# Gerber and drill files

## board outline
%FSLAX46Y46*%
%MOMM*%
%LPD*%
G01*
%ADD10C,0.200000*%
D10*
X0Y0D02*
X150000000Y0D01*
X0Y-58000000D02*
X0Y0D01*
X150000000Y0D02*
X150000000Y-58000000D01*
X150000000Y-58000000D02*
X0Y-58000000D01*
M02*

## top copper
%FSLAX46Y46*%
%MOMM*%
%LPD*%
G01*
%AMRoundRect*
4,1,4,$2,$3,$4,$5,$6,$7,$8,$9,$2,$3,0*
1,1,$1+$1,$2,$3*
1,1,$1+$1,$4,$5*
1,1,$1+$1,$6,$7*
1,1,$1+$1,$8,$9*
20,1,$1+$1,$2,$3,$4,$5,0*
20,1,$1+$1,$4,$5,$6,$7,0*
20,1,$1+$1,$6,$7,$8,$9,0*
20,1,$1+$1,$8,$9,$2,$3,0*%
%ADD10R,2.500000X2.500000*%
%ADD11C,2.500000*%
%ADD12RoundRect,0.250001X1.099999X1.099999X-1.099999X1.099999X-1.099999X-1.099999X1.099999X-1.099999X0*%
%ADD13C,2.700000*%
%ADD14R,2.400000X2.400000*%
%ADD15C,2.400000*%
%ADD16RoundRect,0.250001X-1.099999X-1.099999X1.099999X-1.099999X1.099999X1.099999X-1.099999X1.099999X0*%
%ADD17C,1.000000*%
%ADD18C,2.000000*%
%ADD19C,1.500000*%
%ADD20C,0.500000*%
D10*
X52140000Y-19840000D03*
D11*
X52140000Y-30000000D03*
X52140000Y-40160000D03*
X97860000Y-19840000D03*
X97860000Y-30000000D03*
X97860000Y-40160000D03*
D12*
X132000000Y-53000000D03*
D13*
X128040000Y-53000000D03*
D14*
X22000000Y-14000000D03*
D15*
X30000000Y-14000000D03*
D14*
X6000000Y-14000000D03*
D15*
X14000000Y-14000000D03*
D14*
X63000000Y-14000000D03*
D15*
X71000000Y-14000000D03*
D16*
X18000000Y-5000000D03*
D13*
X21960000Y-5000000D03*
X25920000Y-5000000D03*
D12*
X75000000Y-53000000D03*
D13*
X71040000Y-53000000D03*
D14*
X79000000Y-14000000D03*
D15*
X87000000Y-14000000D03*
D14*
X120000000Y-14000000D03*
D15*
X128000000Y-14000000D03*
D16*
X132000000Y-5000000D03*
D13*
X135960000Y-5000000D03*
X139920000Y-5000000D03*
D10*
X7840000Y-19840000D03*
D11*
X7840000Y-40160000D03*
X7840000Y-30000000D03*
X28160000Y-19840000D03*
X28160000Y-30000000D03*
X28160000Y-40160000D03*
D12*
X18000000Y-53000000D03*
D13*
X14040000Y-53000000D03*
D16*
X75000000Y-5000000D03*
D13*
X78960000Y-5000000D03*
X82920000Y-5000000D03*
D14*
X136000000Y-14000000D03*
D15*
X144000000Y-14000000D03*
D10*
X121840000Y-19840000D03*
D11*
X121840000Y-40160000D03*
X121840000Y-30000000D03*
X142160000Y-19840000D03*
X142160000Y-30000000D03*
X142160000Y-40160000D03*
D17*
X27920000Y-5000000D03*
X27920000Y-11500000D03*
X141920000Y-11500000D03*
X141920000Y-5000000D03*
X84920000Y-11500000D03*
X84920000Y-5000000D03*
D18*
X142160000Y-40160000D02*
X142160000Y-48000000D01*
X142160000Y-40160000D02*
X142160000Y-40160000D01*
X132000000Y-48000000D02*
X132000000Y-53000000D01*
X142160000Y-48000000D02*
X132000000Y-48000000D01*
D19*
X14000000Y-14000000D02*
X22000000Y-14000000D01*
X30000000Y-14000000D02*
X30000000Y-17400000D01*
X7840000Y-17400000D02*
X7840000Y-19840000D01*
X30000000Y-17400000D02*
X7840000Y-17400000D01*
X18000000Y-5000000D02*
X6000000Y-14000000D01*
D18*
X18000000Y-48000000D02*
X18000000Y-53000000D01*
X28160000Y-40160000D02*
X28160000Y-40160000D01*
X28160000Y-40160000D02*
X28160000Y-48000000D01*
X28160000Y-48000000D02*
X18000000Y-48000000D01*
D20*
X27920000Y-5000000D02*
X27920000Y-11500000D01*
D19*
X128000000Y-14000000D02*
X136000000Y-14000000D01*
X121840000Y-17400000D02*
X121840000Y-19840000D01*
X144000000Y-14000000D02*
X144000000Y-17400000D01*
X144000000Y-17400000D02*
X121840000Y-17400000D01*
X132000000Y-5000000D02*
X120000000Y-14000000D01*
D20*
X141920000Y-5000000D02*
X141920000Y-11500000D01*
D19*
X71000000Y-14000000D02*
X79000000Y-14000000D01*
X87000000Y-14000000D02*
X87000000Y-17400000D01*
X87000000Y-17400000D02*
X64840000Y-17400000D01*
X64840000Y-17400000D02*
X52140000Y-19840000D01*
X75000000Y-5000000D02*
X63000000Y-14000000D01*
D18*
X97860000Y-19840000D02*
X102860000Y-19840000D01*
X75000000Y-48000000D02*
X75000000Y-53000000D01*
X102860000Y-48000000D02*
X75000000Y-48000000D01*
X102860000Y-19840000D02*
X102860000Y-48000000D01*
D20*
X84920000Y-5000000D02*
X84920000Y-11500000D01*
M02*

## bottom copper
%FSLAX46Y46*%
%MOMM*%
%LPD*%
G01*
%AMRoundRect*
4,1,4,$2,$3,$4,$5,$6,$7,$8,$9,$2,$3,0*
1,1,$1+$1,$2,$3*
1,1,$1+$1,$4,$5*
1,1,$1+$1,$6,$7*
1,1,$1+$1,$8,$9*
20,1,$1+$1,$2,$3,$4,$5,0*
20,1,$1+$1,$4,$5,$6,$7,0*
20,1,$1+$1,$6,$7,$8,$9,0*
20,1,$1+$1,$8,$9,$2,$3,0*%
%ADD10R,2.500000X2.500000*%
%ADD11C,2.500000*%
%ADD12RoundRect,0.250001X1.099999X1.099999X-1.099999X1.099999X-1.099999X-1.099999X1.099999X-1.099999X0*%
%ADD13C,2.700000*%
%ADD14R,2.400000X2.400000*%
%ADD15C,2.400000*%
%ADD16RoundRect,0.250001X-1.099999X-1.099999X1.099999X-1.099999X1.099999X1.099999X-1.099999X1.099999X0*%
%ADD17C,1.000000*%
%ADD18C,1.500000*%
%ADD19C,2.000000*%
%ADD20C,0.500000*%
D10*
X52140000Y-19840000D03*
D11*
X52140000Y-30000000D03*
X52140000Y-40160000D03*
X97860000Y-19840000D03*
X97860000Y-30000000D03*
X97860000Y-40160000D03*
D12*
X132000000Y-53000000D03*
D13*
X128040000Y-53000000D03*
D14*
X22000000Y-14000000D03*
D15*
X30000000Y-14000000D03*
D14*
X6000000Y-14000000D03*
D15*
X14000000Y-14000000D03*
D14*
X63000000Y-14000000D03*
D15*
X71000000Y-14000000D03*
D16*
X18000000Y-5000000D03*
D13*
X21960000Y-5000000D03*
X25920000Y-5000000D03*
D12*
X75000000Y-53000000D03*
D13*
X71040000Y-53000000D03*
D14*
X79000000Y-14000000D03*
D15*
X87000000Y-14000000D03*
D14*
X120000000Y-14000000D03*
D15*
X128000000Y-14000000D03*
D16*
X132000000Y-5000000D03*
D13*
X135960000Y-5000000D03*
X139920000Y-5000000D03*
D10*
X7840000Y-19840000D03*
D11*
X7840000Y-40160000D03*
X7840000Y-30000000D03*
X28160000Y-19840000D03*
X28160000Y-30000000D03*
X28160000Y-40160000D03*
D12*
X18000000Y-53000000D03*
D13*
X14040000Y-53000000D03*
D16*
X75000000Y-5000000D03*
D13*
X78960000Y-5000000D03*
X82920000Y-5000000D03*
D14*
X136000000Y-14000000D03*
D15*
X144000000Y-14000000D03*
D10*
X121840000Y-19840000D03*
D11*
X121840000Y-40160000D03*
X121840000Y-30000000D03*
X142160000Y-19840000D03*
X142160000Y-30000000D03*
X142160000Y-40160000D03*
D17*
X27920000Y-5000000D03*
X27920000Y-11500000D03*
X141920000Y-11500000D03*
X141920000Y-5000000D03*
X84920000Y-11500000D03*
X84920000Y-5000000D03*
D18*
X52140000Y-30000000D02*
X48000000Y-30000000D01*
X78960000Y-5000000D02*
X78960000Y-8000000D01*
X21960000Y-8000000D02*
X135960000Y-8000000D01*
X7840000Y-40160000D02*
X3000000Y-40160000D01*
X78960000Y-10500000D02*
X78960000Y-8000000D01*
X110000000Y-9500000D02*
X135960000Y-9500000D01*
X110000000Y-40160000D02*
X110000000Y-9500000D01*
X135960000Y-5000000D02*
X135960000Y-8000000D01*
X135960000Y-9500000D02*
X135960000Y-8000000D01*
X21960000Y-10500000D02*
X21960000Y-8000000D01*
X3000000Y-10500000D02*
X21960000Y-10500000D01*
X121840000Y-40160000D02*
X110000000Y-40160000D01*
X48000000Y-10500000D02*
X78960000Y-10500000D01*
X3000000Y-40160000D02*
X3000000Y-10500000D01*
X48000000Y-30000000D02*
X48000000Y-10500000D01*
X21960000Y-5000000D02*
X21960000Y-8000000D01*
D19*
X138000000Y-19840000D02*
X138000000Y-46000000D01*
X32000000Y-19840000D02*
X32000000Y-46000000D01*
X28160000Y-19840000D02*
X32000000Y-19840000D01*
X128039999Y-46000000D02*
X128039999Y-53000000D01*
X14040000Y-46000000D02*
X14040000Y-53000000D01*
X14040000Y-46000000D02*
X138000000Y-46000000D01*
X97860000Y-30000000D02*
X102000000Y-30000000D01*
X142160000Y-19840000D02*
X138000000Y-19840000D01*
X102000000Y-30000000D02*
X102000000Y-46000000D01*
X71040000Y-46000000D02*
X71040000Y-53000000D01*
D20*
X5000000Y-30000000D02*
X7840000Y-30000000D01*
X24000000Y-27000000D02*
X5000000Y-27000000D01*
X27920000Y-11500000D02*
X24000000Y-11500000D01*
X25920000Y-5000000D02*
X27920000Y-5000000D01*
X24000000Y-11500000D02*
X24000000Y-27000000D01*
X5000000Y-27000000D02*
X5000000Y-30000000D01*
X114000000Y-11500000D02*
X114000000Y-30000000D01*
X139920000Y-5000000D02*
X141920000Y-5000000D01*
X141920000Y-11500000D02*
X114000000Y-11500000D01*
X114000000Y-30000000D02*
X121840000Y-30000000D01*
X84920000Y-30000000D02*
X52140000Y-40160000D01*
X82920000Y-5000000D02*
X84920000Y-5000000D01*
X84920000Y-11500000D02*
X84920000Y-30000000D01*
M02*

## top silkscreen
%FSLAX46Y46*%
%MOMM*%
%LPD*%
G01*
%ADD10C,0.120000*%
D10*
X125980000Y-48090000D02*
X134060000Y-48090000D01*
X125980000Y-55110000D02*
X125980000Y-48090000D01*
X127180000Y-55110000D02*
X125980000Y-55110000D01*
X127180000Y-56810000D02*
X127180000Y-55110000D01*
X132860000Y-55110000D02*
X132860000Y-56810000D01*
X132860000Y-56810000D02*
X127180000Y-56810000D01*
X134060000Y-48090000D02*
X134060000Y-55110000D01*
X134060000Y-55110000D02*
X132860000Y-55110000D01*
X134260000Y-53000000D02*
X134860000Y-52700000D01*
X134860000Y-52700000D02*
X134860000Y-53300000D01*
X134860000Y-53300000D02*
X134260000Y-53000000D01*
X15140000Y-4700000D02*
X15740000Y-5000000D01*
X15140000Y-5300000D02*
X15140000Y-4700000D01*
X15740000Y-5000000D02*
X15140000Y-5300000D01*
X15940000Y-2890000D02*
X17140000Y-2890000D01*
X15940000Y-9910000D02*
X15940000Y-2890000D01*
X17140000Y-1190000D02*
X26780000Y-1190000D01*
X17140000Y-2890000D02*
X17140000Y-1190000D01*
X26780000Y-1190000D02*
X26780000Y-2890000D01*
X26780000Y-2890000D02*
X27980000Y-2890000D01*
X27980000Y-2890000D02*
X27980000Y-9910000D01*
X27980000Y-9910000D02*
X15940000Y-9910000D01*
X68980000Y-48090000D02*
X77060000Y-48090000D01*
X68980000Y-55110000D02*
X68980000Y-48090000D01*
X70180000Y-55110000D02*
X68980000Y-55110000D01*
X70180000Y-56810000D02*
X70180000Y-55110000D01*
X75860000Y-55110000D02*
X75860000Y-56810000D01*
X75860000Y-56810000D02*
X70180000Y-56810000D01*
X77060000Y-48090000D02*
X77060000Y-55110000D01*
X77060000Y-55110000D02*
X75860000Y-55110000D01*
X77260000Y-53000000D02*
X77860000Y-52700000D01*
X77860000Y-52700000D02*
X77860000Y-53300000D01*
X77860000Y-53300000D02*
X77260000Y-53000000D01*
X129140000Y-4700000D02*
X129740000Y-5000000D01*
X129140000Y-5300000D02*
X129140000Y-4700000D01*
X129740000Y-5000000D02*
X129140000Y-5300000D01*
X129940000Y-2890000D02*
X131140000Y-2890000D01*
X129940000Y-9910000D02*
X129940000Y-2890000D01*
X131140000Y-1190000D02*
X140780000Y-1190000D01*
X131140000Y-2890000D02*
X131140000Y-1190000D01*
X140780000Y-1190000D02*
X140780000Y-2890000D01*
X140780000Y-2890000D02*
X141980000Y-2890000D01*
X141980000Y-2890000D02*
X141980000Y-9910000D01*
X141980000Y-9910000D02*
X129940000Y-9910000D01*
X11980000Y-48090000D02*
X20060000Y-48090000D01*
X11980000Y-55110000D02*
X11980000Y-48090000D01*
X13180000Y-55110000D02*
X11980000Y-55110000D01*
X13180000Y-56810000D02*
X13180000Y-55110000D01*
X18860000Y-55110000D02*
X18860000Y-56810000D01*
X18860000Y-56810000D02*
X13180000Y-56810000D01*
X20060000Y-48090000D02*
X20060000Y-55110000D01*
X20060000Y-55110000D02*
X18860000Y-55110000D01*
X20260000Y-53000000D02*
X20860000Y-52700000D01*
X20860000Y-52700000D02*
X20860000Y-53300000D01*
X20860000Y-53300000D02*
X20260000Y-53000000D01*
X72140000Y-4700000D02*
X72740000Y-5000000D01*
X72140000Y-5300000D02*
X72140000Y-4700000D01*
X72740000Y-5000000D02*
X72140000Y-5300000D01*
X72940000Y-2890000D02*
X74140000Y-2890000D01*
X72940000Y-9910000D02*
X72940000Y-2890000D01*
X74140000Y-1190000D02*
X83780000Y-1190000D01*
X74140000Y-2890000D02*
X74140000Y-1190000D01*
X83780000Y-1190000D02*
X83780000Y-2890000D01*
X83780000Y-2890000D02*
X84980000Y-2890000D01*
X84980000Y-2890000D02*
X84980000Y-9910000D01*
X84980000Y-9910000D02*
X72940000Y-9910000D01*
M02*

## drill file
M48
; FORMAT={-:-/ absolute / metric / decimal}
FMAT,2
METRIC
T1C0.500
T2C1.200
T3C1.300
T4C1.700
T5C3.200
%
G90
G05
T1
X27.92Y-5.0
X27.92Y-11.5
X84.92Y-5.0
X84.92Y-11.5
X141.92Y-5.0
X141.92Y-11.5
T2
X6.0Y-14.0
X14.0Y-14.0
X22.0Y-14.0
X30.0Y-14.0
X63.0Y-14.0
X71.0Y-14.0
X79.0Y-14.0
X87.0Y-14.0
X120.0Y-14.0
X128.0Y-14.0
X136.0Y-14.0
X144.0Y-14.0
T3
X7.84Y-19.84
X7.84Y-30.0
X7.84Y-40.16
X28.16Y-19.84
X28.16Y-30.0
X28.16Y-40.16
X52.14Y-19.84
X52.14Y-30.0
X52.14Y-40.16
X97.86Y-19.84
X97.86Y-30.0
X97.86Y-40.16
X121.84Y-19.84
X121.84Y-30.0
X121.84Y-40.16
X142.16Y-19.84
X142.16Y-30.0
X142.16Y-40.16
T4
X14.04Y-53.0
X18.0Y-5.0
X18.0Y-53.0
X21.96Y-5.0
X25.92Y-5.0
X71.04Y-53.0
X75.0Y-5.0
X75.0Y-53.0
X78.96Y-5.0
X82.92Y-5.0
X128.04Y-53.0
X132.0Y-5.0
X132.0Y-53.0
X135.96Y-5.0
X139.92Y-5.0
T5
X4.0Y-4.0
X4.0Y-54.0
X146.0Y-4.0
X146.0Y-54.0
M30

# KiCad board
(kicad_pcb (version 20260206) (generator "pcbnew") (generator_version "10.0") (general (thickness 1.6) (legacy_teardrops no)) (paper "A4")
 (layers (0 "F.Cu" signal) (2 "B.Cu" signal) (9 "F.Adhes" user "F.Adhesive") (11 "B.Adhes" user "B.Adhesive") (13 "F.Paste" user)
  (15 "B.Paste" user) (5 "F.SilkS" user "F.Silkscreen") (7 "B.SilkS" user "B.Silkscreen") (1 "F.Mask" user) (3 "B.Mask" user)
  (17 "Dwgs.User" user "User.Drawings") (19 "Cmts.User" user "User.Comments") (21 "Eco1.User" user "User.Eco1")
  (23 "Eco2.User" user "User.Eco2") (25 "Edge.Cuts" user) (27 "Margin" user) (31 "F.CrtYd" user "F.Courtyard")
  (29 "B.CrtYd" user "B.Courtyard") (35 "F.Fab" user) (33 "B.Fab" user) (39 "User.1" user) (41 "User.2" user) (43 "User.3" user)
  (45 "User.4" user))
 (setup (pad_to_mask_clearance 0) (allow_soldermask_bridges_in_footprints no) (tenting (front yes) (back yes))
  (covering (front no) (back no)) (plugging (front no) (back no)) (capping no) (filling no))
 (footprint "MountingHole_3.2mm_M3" (layer "F.Cu") (at 4 4)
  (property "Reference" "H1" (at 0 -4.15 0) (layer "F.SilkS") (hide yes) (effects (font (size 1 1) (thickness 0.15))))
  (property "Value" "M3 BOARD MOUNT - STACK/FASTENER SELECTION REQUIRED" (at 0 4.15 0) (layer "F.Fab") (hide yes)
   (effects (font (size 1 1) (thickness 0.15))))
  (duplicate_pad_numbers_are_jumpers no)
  (pad "" np_thru_hole circle (at 0 0) (size 3.2 3.2) (drill 3.2) (layers "*.Cu")))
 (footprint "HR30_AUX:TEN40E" (layer "F.Cu") (at 75 30)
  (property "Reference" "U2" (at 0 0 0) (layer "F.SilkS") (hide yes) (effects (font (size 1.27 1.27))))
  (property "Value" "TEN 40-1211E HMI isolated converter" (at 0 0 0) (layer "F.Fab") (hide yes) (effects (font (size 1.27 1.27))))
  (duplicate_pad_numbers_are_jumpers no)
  (pad "1" thru_hole rect (at -22.86 -10.16) (size 2.5 2.5) (drill 1.3) (layers "*.Cu") (remove_unused_layers no) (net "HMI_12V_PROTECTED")
   (thermal_bridge_angle 45))
  (pad "2" thru_hole circle (at -22.86 0) (size 2.5 2.5) (drill 1.3) (layers "*.Cu") (remove_unused_layers no) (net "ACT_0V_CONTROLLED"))
  (pad "3" thru_hole circle (at -22.86 10.16) (size 2.5 2.5) (drill 1.3) (layers "*.Cu") (remove_unused_layers no) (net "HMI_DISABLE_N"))
  (pad "4" thru_hole circle (at 22.86 -10.16) (size 2.5 2.5) (drill 1.3) (layers "*.Cu") (remove_unused_layers no) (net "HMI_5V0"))
  (pad "5" thru_hole circle (at 22.86 0) (size 2.5 2.5) (drill 1.3) (layers "*.Cu") (remove_unused_layers no) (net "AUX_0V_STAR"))
  (pad "6" thru_hole circle (at 22.86 10.16) (size 2.5 2.5) (drill 1.3) (layers "*.Cu") (remove_unused_layers no)))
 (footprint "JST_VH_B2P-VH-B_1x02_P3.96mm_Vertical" (layer "F.Cu") (at 132 53 180)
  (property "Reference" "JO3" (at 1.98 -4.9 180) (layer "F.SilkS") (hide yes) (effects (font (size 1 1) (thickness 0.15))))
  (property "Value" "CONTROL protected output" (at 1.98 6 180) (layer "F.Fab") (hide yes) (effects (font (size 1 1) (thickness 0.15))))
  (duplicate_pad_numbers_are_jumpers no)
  (fp_line (start 6.02 4.91) (end -2.06 4.91) (stroke (width 0.12) (type solid)) (layer "F.SilkS"))
  (fp_line (start 6.02 -2.11) (end 6.02 4.91) (stroke (width 0.12) (type solid)) (layer "F.SilkS"))
  (fp_line (start 4.82 -2.11) (end 6.02 -2.11) (stroke (width 0.12) (type solid)) (layer "F.SilkS"))
  (fp_line (start 4.82 -3.81) (end 4.82 -2.11) (stroke (width 0.12) (type solid)) (layer "F.SilkS"))
  (fp_line (start -0.86 -2.11) (end -0.86 -3.81) (stroke (width 0.12) (type solid)) (layer "F.SilkS"))
  (fp_line (start -0.86 -3.81) (end 4.82 -3.81) (stroke (width 0.12) (type solid)) (layer "F.SilkS"))
  (fp_line (start -2.06 4.91) (end -2.06 -2.11) (stroke (width 0.12) (type solid)) (layer "F.SilkS"))
  (fp_line (start -2.06 -2.11) (end -0.86 -2.11) (stroke (width 0.12) (type solid)) (layer "F.SilkS"))
  (fp_line (start -2.26 0) (end -2.86 0.3) (stroke (width 0.12) (type solid)) (layer "F.SilkS"))
  (fp_line (start -2.86 0.3) (end -2.86 -0.3) (stroke (width 0.12) (type solid)) (layer "F.SilkS"))
  (fp_line (start -2.86 -0.3) (end -2.26 0) (stroke (width 0.12) (type solid)) (layer "F.SilkS"))
  (pad "1" thru_hole roundrect (at 0 0 180) (size 2.7 2.7) (drill 1.7) (layers "*.Cu") (remove_unused_layers no) (roundrect_rratio 0.092593)
   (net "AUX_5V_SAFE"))
  (pad "2" thru_hole circle (at 3.96 0 180) (size 2.7 2.7) (drill 1.7) (layers "*.Cu") (remove_unused_layers no) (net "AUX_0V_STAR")))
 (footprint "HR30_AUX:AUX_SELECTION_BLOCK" (layer "F.Cu") (at 26 14)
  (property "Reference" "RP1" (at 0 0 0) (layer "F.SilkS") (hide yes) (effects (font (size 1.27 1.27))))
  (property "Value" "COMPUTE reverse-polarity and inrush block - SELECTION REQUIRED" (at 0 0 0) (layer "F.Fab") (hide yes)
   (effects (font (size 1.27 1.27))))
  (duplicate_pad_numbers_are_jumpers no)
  (pad "1" thru_hole rect (at -4 0) (size 2.4 2.4) (drill 1.2) (layers "*.Cu") (remove_unused_layers no) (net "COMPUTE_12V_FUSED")
   (thermal_bridge_angle 45))
  (pad "2" thru_hole circle (at 4 0) (size 2.4 2.4) (drill 1.2) (layers "*.Cu") (remove_unused_layers no) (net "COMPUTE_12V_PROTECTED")))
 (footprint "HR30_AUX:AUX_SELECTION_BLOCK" (layer "F.Cu") (at 10 14)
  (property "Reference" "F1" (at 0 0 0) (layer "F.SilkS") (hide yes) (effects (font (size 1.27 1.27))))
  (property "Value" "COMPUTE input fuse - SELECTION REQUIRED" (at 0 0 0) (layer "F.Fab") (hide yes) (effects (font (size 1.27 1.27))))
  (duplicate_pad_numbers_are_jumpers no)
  (pad "1" thru_hole rect (at -4 0) (size 2.4 2.4) (drill 1.2) (layers "*.Cu") (remove_unused_layers no) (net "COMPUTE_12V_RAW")
   (thermal_bridge_angle 45))
  (pad "2" thru_hole circle (at 4 0) (size 2.4 2.4) (drill 1.2) (layers "*.Cu") (remove_unused_layers no) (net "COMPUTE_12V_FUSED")))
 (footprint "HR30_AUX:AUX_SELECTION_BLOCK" (layer "F.Cu") (at 67 14)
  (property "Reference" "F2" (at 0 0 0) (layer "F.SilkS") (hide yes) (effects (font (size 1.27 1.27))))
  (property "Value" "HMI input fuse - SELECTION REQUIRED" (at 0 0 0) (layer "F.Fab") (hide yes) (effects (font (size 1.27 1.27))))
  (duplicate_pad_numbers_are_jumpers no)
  (pad "1" thru_hole rect (at -4 0) (size 2.4 2.4) (drill 1.2) (layers "*.Cu") (remove_unused_layers no) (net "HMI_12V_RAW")
   (thermal_bridge_angle 45))
  (pad "2" thru_hole circle (at 4 0) (size 2.4 2.4) (drill 1.2) (layers "*.Cu") (remove_unused_layers no) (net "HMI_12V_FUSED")))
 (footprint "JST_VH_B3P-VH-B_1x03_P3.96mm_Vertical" (layer "F.Cu") (at 18 5)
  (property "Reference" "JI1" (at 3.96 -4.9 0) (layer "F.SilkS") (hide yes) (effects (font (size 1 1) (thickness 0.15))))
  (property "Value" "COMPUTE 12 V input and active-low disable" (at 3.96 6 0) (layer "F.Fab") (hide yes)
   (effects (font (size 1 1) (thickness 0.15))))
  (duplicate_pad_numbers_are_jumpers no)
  (fp_line (start -2.86 -0.3) (end -2.26 0) (stroke (width 0.12) (type solid)) (layer "F.SilkS"))
  (fp_line (start -2.86 0.3) (end -2.86 -0.3) (stroke (width 0.12) (type solid)) (layer "F.SilkS"))
  (fp_line (start -2.26 0) (end -2.86 0.3) (stroke (width 0.12) (type solid)) (layer "F.SilkS"))
  (fp_line (start -2.06 -2.11) (end -0.86 -2.11) (stroke (width 0.12) (type solid)) (layer "F.SilkS"))
  (fp_line (start -2.06 4.91) (end -2.06 -2.11) (stroke (width 0.12) (type solid)) (layer "F.SilkS"))
  (fp_line (start -0.86 -3.81) (end 8.78 -3.81) (stroke (width 0.12) (type solid)) (layer "F.SilkS"))
  (fp_line (start -0.86 -2.11) (end -0.86 -3.81) (stroke (width 0.12) (type solid)) (layer "F.SilkS"))
  (fp_line (start 8.78 -3.81) (end 8.78 -2.11) (stroke (width 0.12) (type solid)) (layer "F.SilkS"))
  (fp_line (start 8.78 -2.11) (end 9.98 -2.11) (stroke (width 0.12) (type solid)) (layer "F.SilkS"))
  (fp_line (start 9.98 -2.11) (end 9.98 4.91) (stroke (width 0.12) (type solid)) (layer "F.SilkS"))
  (fp_line (start 9.98 4.91) (end -2.06 4.91) (stroke (width 0.12) (type solid)) (layer "F.SilkS"))
  (pad "1" thru_hole roundrect (at 0 0) (size 2.7 2.7) (drill 1.7) (layers "*.Cu") (remove_unused_layers no) (roundrect_rratio 0.092593)
   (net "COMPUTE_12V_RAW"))
  (pad "2" thru_hole circle (at 3.96 0) (size 2.7 2.7) (drill 1.7) (layers "*.Cu") (remove_unused_layers no) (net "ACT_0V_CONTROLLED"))
  (pad "3" thru_hole circle (at 7.92 0) (size 2.7 2.7) (drill 1.7) (layers "*.Cu") (remove_unused_layers no) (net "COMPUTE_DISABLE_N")))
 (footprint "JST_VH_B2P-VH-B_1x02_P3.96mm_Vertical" (layer "F.Cu") (at 75 53 180)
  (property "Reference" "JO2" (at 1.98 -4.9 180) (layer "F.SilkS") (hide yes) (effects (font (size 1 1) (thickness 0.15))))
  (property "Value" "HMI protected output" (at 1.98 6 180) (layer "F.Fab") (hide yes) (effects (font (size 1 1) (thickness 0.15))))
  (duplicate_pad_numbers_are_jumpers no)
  (fp_line (start 6.02 4.91) (end -2.06 4.91) (stroke (width 0.12) (type solid)) (layer "F.SilkS"))
  (fp_line (start 6.02 -2.11) (end 6.02 4.91) (stroke (width 0.12) (type solid)) (layer "F.SilkS"))
  (fp_line (start 4.82 -2.11) (end 6.02 -2.11) (stroke (width 0.12) (type solid)) (layer "F.SilkS"))
  (fp_line (start 4.82 -3.81) (end 4.82 -2.11) (stroke (width 0.12) (type solid)) (layer "F.SilkS"))
  (fp_line (start -0.86 -2.11) (end -0.86 -3.81) (stroke (width 0.12) (type solid)) (layer "F.SilkS"))
  (fp_line (start -0.86 -3.81) (end 4.82 -3.81) (stroke (width 0.12) (type solid)) (layer "F.SilkS"))
  (fp_line (start -2.06 4.91) (end -2.06 -2.11) (stroke (width 0.12) (type solid)) (layer "F.SilkS"))
  (fp_line (start -2.06 -2.11) (end -0.86 -2.11) (stroke (width 0.12) (type solid)) (layer "F.SilkS"))
  (fp_line (start -2.26 0) (end -2.86 0.3) (stroke (width 0.12) (type solid)) (layer "F.SilkS"))
  (fp_line (start -2.86 0.3) (end -2.86 -0.3) (stroke (width 0.12) (type solid)) (layer "F.SilkS"))
  (fp_line (start -2.86 -0.3) (end -2.26 0) (stroke (width 0.12) (type solid)) (layer "F.SilkS"))
  (pad "1" thru_hole roundrect (at 0 0 180) (size 2.7 2.7) (drill 1.7) (layers "*.Cu") (remove_unused_layers no) (roundrect_rratio 0.092593)
   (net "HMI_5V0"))
  (pad "2" thru_hole circle (at 3.96 0 180) (size 2.7 2.7) (drill 1.7) (layers "*.Cu") (remove_unused_layers no) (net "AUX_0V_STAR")))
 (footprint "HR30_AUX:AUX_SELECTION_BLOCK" (layer "F.Cu") (at 83 14)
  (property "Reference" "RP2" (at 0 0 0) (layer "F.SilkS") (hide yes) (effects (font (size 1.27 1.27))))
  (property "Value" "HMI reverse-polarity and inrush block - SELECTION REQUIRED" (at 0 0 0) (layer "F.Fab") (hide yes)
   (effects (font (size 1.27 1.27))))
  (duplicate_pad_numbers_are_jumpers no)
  (pad "1" thru_hole rect (at -4 0) (size 2.4 2.4) (drill 1.2) (layers "*.Cu") (remove_unused_layers no) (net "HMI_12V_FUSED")
   (thermal_bridge_angle 45))
  (pad "2" thru_hole circle (at 4 0) (size 2.4 2.4) (drill 1.2) (layers "*.Cu") (remove_unused_layers no) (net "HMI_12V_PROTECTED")))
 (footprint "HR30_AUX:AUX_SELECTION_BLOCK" (layer "F.Cu") (at 124 14)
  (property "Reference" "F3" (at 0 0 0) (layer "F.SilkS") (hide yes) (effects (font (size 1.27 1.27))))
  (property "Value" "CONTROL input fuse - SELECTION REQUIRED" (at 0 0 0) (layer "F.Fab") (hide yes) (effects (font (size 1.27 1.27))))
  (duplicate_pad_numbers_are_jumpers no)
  (pad "1" thru_hole rect (at -4 0) (size 2.4 2.4) (drill 1.2) (layers "*.Cu") (remove_unused_layers no) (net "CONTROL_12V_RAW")
   (thermal_bridge_angle 45))
  (pad "2" thru_hole circle (at 4 0) (size 2.4 2.4) (drill 1.2) (layers "*.Cu") (remove_unused_layers no) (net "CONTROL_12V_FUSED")))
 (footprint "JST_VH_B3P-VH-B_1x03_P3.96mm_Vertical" (layer "F.Cu") (at 132 5)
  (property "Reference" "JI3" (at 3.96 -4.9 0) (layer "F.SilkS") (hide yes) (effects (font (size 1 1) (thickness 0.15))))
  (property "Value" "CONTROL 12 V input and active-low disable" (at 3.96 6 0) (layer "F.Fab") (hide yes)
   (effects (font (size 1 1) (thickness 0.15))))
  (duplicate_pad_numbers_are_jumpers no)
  (fp_line (start -2.86 -0.3) (end -2.26 0) (stroke (width 0.12) (type solid)) (layer "F.SilkS"))
  (fp_line (start -2.86 0.3) (end -2.86 -0.3) (stroke (width 0.12) (type solid)) (layer "F.SilkS"))
  (fp_line (start -2.26 0) (end -2.86 0.3) (stroke (width 0.12) (type solid)) (layer "F.SilkS"))
  (fp_line (start -2.06 -2.11) (end -0.86 -2.11) (stroke (width 0.12) (type solid)) (layer "F.SilkS"))
  (fp_line (start -2.06 4.91) (end -2.06 -2.11) (stroke (width 0.12) (type solid)) (layer "F.SilkS"))
  (fp_line (start -0.86 -3.81) (end 8.78 -3.81) (stroke (width 0.12) (type solid)) (layer "F.SilkS"))
  (fp_line (start -0.86 -2.11) (end -0.86 -3.81) (stroke (width 0.12) (type solid)) (layer "F.SilkS"))
  (fp_line (start 8.78 -3.81) (end 8.78 -2.11) (stroke (width 0.12) (type solid)) (layer "F.SilkS"))
  (fp_line (start 8.78 -2.11) (end 9.98 -2.11) (stroke (width 0.12) (type solid)) (layer "F.SilkS"))
  (fp_line (start 9.98 -2.11) (end 9.98 4.91) (stroke (width 0.12) (type solid)) (layer "F.SilkS"))
  (fp_line (start 9.98 4.91) (end -2.06 4.91) (stroke (width 0.12) (type solid)) (layer "F.SilkS"))
  (pad "1" thru_hole roundrect (at 0 0) (size 2.7 2.7) (drill 1.7) (layers "*.Cu") (remove_unused_layers no) (roundrect_rratio 0.092593)
   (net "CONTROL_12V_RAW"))
  (pad "2" thru_hole circle (at 3.96 0) (size 2.7 2.7) (drill 1.7) (layers "*.Cu") (remove_unused_layers no) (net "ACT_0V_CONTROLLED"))
  (pad "3" thru_hole circle (at 7.92 0) (size 2.7 2.7) (drill 1.7) (layers "*.Cu") (remove_unused_layers no) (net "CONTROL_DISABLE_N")))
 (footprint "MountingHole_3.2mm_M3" (layer "F.Cu") (at 4 54)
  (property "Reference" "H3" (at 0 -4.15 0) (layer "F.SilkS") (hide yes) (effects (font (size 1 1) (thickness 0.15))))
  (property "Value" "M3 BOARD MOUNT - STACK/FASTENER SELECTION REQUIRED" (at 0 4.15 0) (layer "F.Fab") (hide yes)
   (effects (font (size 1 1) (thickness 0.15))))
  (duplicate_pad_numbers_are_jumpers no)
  (pad "" np_thru_hole circle (at 0 0) (size 3.2 3.2) (drill 3.2) (layers "*.Cu")))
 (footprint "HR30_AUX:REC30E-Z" (layer "F.Cu") (at 18 30)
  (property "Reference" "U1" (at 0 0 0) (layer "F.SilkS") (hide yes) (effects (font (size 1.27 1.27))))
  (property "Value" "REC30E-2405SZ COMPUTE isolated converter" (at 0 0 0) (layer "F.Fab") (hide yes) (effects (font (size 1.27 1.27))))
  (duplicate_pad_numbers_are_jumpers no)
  (pad "1" thru_hole rect (at -10.16 -10.16) (size 2.5 2.5) (drill 1.3) (layers "*.Cu") (remove_unused_layers no)
   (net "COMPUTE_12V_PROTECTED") (thermal_bridge_angle 45))
  (pad "2" thru_hole circle (at -10.16 10.16) (size 2.5 2.5) (drill 1.3) (layers "*.Cu") (remove_unused_layers no) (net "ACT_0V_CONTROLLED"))
  (pad "3" thru_hole circle (at -10.16 0) (size 2.5 2.5) (drill 1.3) (layers "*.Cu") (remove_unused_layers no) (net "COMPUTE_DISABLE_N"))
  (pad "4" thru_hole circle (at 10.16 -10.16) (size 2.5 2.5) (drill 1.3) (layers "*.Cu") (remove_unused_layers no) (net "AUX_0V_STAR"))
  (pad "5" thru_hole circle (at 10.16 0) (size 2.5 2.5) (drill 1.3) (layers "*.Cu") (remove_unused_layers no))
  (pad "6" thru_hole circle (at 10.16 10.16) (size 2.5 2.5) (drill 1.3) (layers "*.Cu") (remove_unused_layers no) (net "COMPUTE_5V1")))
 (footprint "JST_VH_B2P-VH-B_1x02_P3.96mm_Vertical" (layer "F.Cu") (at 18 53 180)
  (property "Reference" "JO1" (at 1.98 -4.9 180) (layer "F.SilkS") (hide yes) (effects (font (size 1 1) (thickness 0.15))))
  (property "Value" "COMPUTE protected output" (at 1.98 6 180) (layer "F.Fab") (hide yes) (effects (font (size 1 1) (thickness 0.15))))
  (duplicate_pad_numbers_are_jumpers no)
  (fp_line (start 6.02 4.91) (end -2.06 4.91) (stroke (width 0.12) (type solid)) (layer "F.SilkS"))
  (fp_line (start 6.02 -2.11) (end 6.02 4.91) (stroke (width 0.12) (type solid)) (layer "F.SilkS"))
  (fp_line (start 4.82 -2.11) (end 6.02 -2.11) (stroke (width 0.12) (type solid)) (layer "F.SilkS"))
  (fp_line (start 4.82 -3.81) (end 4.82 -2.11) (stroke (width 0.12) (type solid)) (layer "F.SilkS"))
  (fp_line (start -0.86 -2.11) (end -0.86 -3.81) (stroke (width 0.12) (type solid)) (layer "F.SilkS"))
  (fp_line (start -0.86 -3.81) (end 4.82 -3.81) (stroke (width 0.12) (type solid)) (layer "F.SilkS"))
  (fp_line (start -2.06 4.91) (end -2.06 -2.11) (stroke (width 0.12) (type solid)) (layer "F.SilkS"))
  (fp_line (start -2.06 -2.11) (end -0.86 -2.11) (stroke (width 0.12) (type solid)) (layer "F.SilkS"))
  (fp_line (start -2.26 0) (end -2.86 0.3) (stroke (width 0.12) (type solid)) (layer "F.SilkS"))
  (fp_line (start -2.86 0.3) (end -2.86 -0.3) (stroke (width 0.12) (type solid)) (layer "F.SilkS"))
  (fp_line (start -2.86 -0.3) (end -2.26 0) (stroke (width 0.12) (type solid)) (layer "F.SilkS"))
  (pad "1" thru_hole roundrect (at 0 0 180) (size 2.7 2.7) (drill 1.7) (layers "*.Cu") (remove_unused_layers no) (roundrect_rratio 0.092593)
   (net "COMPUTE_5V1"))
  (pad "2" thru_hole circle (at 3.96 0 180) (size 2.7 2.7) (drill 1.7) (layers "*.Cu") (remove_unused_layers no) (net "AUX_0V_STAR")))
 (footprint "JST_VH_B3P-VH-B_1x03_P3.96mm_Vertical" (layer "F.Cu") (at 75 5)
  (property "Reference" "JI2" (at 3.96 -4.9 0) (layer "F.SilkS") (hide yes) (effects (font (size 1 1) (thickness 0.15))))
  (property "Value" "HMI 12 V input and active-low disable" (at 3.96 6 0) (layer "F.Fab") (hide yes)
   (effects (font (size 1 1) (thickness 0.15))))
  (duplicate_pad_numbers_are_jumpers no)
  (fp_line (start -2.86 -0.3) (end -2.26 0) (stroke (width 0.12) (type solid)) (layer "F.SilkS"))
  (fp_line (start -2.86 0.3) (end -2.86 -0.3) (stroke (width 0.12) (type solid)) (layer "F.SilkS"))
  (fp_line (start -2.26 0) (end -2.86 0.3) (stroke (width 0.12) (type solid)) (layer "F.SilkS"))
  (fp_line (start -2.06 -2.11) (end -0.86 -2.11) (stroke (width 0.12) (type solid)) (layer "F.SilkS"))
  (fp_line (start -2.06 4.91) (end -2.06 -2.11) (stroke (width 0.12) (type solid)) (layer "F.SilkS"))
  (fp_line (start -0.86 -3.81) (end 8.78 -3.81) (stroke (width 0.12) (type solid)) (layer "F.SilkS"))
  (fp_line (start -0.86 -2.11) (end -0.86 -3.81) (stroke (width 0.12) (type solid)) (layer "F.SilkS"))
  (fp_line (start 8.78 -3.81) (end 8.78 -2.11) (stroke (width 0.12) (type solid)) (layer "F.SilkS"))
  (fp_line (start 8.78 -2.11) (end 9.98 -2.11) (stroke (width 0.12) (type solid)) (layer "F.SilkS"))
  (fp_line (start 9.98 -2.11) (end 9.98 4.91) (stroke (width 0.12) (type solid)) (layer "F.SilkS"))
  (fp_line (start 9.98 4.91) (end -2.06 4.91) (stroke (width 0.12) (type solid)) (layer "F.SilkS"))
  (pad "1" thru_hole roundrect (at 0 0) (size 2.7 2.7) (drill 1.7) (layers "*.Cu") (remove_unused_layers no) (roundrect_rratio 0.092593)
   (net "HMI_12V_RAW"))
  (pad "2" thru_hole circle (at 3.96 0) (size 2.7 2.7) (drill 1.7) (layers "*.Cu") (remove_unused_layers no) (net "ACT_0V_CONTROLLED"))
  (pad "3" thru_hole circle (at 7.92 0) (size 2.7 2.7) (drill 1.7) (layers "*.Cu") (remove_unused_layers no) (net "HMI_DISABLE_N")))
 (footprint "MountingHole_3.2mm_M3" (layer "F.Cu") (at 146 54)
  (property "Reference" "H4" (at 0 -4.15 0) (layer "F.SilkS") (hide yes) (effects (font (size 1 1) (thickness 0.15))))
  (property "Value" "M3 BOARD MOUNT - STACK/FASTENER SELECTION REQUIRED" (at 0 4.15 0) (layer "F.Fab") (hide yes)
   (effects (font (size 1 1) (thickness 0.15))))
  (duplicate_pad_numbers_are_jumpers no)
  (pad "" np_thru_hole circle (at 0 0) (size 3.2 3.2) (drill 3.2) (layers "*.Cu")))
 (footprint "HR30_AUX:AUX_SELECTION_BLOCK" (layer "F.Cu") (at 140 14)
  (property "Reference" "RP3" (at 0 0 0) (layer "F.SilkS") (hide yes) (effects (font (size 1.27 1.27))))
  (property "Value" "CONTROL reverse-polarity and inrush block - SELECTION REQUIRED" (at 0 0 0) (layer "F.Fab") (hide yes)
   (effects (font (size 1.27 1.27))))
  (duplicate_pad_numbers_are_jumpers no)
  (pad "1" thru_hole rect (at -4 0) (size 2.4 2.4) (drill 1.2) (layers "*.Cu") (remove_unused_layers no) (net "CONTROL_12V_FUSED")
   (thermal_bridge_angle 45))
  (pad "2" thru_hole circle (at 4 0) (size 2.4 2.4) (drill 1.2) (layers "*.Cu") (remove_unused_layers no) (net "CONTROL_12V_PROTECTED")))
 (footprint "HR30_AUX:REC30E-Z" (layer "F.Cu") (at 132 30)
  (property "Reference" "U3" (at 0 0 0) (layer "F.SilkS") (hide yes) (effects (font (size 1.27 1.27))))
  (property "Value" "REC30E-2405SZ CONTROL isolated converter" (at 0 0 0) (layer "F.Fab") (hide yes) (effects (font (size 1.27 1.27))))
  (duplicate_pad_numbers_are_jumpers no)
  (pad "1" thru_hole rect (at -10.16 -10.16) (size 2.5 2.5) (drill 1.3) (layers "*.Cu") (remove_unused_layers no)
   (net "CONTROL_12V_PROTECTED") (thermal_bridge_angle 45))
  (pad "2" thru_hole circle (at -10.16 10.16) (size 2.5 2.5) (drill 1.3) (layers "*.Cu") (remove_unused_layers no) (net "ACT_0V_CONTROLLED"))
  (pad "3" thru_hole circle (at -10.16 0) (size 2.5 2.5) (drill 1.3) (layers "*.Cu") (remove_unused_layers no) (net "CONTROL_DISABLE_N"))
  (pad "4" thru_hole circle (at 10.16 -10.16) (size 2.5 2.5) (drill 1.3) (layers "*.Cu") (remove_unused_layers no) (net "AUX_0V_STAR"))
  (pad "5" thru_hole circle (at 10.16 0) (size 2.5 2.5) (drill 1.3) (layers "*.Cu") (remove_unused_layers no))
  (pad "6" thru_hole circle (at 10.16 10.16) (size 2.5 2.5) (drill 1.3) (layers "*.Cu") (remove_unused_layers no) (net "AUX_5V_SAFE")))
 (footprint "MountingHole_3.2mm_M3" (layer "F.Cu") (at 146 4)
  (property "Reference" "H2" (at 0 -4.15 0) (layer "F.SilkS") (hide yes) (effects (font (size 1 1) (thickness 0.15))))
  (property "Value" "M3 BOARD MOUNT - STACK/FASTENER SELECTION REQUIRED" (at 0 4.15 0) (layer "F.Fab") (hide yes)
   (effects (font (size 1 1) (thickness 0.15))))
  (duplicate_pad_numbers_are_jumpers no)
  (pad "" np_thru_hole circle (at 0 0) (size 3.2 3.2) (drill 3.2) (layers "*.Cu")))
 (gr_line (start 0 0) (end 150 0) (stroke (width 0.2) (type default)) (layer "Edge.Cuts"))
 (gr_line (start 0 58) (end 0 0) (stroke (width 0.2) (type default)) (layer "Edge.Cuts"))
 (gr_line (start 150 0) (end 150 58) (stroke (width 0.2) (type default)) (layer "Edge.Cuts"))
 (gr_line (start 150 58) (end 0 58) (stroke (width 0.2) (type default)) (layer "Edge.Cuts"))
 (segment (start 52.14 30) (end 48 30) (width 1.5) (layer "B.Cu") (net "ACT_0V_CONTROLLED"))
 (segment (start 78.96 5) (end 78.96 8) (width 1.5) (layer "B.Cu") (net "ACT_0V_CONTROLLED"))
 (segment (start 21.96 8) (end 135.96 8) (width 1.5) (layer "B.Cu") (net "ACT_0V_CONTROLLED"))
 (segment (start 7.84 40.16) (end 3 40.16) (width 1.5) (layer "B.Cu") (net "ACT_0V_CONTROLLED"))
 (segment (start 78.96 10.5) (end 78.96 8) (width 1.5) (layer "B.Cu") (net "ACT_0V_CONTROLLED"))
 (segment (start 110 9.5) (end 135.96 9.5) (width 1.5) (layer "B.Cu") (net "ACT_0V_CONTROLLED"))
 (segment (start 110 40.16) (end 110 9.5) (width 1.5) (layer "B.Cu") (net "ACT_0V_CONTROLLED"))
 (segment (start 135.96 5) (end 135.96 8) (width 1.5) (layer "B.Cu") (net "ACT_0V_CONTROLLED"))
 (segment (start 135.96 9.5) (end 135.96 8) (width 1.5) (layer "B.Cu") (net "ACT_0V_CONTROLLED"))
 (segment (start 21.96 10.5) (end 21.96 8) (width 1.5) (layer "B.Cu") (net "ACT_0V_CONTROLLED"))
 (segment (start 3 10.5) (end 21.96 10.5) (width 1.5) (layer "B.Cu") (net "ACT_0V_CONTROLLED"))
 (segment (start 121.84 40.16) (end 110 40.16) (width 1.5) (layer "B.Cu") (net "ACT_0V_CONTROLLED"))
 (segment (start 48 10.5) (end 78.96 10.5) (width 1.5) (layer "B.Cu") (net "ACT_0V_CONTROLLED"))
 (segment (start 3 40.16) (end 3 10.5) (width 1.5) (layer "B.Cu") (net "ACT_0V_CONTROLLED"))
 (segment (start 48 30) (end 48 10.5) (width 1.5) (layer "B.Cu") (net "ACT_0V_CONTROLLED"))
 (segment (start 21.96 5) (end 21.96 8) (width 1.5) (layer "B.Cu") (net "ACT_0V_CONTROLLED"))
 (segment (start 138 19.84) (end 138 46) (width 2) (layer "B.Cu") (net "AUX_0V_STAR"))
 (segment (start 32 19.84) (end 32 46) (width 2) (layer "B.Cu") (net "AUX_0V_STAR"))
 (segment (start 28.16 19.84) (end 32 19.84) (width 2) (layer "B.Cu") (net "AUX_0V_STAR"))
 (segment (start 128.039999 46) (end 128.039999 53) (width 2) (layer "B.Cu") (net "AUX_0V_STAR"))
 (segment (start 14.04 46) (end 14.04 53) (width 2) (layer "B.Cu") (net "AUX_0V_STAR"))
 (segment (start 14.04 46) (end 138 46) (width 2) (layer "B.Cu") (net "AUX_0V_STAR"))
 (segment (start 97.86 30) (end 102 30) (width 2) (layer "B.Cu") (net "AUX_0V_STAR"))
 (segment (start 142.16 19.84) (end 138 19.84) (width 2) (layer "B.Cu") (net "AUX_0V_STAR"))
 (segment (start 102 30) (end 102 46) (width 2) (layer "B.Cu") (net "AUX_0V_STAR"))
 (segment (start 71.04 46) (end 71.04 53) (width 2) (layer "B.Cu") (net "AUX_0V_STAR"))
 (segment (start 142.16 40.16) (end 142.16 48) (width 2) (layer "F.Cu") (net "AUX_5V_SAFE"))
 (segment (start 142.16 40.16) (end 142.16 40.16) (width 2) (layer "F.Cu") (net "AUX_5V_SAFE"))
 (segment (start 132 48) (end 132 53) (width 2) (layer "F.Cu") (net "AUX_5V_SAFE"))
 (segment (start 142.16 48) (end 132 48) (width 2) (layer "F.Cu") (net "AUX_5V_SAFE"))
 (segment (start 14 14) (end 22 14) (width 1.5) (layer "F.Cu") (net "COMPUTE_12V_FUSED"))
 (segment (start 30 14) (end 30 17.4) (width 1.5) (layer "F.Cu") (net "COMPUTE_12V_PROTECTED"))
 (segment (start 7.84 17.4) (end 7.84 19.84) (width 1.5) (layer "F.Cu") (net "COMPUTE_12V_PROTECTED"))
 (segment (start 30 17.4) (end 7.84 17.4) (width 1.5) (layer "F.Cu") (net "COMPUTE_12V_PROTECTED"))
 (segment (start 18 5) (end 6 14) (width 1.5) (layer "F.Cu") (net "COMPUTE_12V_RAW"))
 (segment (start 18 48) (end 18 53) (width 2) (layer "F.Cu") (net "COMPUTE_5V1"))
 (segment (start 28.16 40.16) (end 28.16 40.16) (width 2) (layer "F.Cu") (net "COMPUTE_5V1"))
 (segment (start 28.16 40.16) (end 28.16 48) (width 2) (layer "F.Cu") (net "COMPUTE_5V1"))
 (segment (start 28.16 48) (end 18 48) (width 2) (layer "F.Cu") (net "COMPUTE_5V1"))
 (segment (start 27.92 5) (end 27.92 11.5) (width 0.5) (layer "F.Cu") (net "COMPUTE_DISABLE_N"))
 (via (at 27.92 5) (size 1) (drill 0.5) (layers "F.Cu" "B.Cu") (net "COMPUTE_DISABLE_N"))
 (via (at 27.92 11.5) (size 1) (drill 0.5) (layers "F.Cu" "B.Cu") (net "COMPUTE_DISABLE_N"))
 (segment (start 5 30) (end 7.84 30) (width 0.5) (layer "B.Cu") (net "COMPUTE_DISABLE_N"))
 (segment (start 24 27) (end 5 27) (width 0.5) (layer "B.Cu") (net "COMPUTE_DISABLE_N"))
 (segment (start 27.92 11.5) (end 24 11.5) (width 0.5) (layer "B.Cu") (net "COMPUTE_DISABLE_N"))
 (segment (start 25.92 5) (end 27.92 5) (width 0.5) (layer "B.Cu") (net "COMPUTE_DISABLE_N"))
 (segment (start 24 11.5) (end 24 27) (width 0.5) (layer "B.Cu") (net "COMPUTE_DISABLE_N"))
 (segment (start 5 27) (end 5 30) (width 0.5) (layer "B.Cu") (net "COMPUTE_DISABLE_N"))
 (segment (start 128 14) (end 136 14) (width 1.5) (layer "F.Cu") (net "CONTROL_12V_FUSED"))
 (segment (start 121.84 17.4) (end 121.84 19.84) (width 1.5) (layer "F.Cu") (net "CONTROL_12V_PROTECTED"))
 (segment (start 144 14) (end 144 17.4) (width 1.5) (layer "F.Cu") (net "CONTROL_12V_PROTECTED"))
 (segment (start 144 17.4) (end 121.84 17.4) (width 1.5) (layer "F.Cu") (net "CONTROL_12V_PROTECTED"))
 (segment (start 132 5) (end 120 14) (width 1.5) (layer "F.Cu") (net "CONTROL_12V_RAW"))
 (segment (start 141.92 5) (end 141.92 11.5) (width 0.5) (layer "F.Cu") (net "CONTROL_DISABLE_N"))
 (via (at 141.92 11.5) (size 1) (drill 0.5) (layers "F.Cu" "B.Cu") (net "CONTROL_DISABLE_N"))
 (via (at 141.92 5) (size 1) (drill 0.5) (layers "F.Cu" "B.Cu") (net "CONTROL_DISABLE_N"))
 (segment (start 114 11.5) (end 114 30) (width 0.5) (layer "B.Cu") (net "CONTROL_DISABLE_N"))
 (segment (start 139.92 5) (end 141.92 5) (width 0.5) (layer "B.Cu") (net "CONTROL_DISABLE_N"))
 (segment (start 141.92 11.5) (end 114 11.5) (width 0.5) (layer "B.Cu") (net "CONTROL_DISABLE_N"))
 (segment (start 114 30) (end 121.84 30) (width 0.5) (layer "B.Cu") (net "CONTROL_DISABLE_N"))
 (segment (start 71 14) (end 79 14) (width 1.5) (layer "F.Cu") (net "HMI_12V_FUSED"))
 (segment (start 87 14) (end 87 17.4) (width 1.5) (layer "F.Cu") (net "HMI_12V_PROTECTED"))
 (segment (start 87 17.4) (end 64.84 17.4) (width 1.5) (layer "F.Cu") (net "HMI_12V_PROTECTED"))
 (segment (start 64.84 17.4) (end 52.14 19.84) (width 1.5) (layer "F.Cu") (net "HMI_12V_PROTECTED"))
 (segment (start 75 5) (end 63 14) (width 1.5) (layer "F.Cu") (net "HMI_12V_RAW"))
 (segment (start 97.86 19.84) (end 102.86 19.84) (width 2) (layer "F.Cu") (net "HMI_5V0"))
 (segment (start 75 48) (end 75 53) (width 2) (layer "F.Cu") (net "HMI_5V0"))
 (segment (start 102.86 48) (end 75 48) (width 2) (layer "F.Cu") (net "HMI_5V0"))
 (segment (start 102.86 19.84) (end 102.86 48) (width 2) (layer "F.Cu") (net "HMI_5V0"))
 (segment (start 84.92 5) (end 84.92 11.5) (width 0.5) (layer "F.Cu") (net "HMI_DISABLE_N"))
 (via (at 84.92 11.5) (size 1) (drill 0.5) (layers "F.Cu" "B.Cu") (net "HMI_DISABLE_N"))
 (via (at 84.92 5) (size 1) (drill 0.5) (layers "F.Cu" "B.Cu") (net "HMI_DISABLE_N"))
 (segment (start 84.92 30) (end 52.14 40.16) (width 0.5) (layer "B.Cu") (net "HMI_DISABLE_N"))
 (segment (start 82.92 5) (end 84.92 5) (width 0.5) (layer "B.Cu") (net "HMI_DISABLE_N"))
 (segment (start 84.92 11.5) (end 84.92 30) (width 0.5) (layer "B.Cu") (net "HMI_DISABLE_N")))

